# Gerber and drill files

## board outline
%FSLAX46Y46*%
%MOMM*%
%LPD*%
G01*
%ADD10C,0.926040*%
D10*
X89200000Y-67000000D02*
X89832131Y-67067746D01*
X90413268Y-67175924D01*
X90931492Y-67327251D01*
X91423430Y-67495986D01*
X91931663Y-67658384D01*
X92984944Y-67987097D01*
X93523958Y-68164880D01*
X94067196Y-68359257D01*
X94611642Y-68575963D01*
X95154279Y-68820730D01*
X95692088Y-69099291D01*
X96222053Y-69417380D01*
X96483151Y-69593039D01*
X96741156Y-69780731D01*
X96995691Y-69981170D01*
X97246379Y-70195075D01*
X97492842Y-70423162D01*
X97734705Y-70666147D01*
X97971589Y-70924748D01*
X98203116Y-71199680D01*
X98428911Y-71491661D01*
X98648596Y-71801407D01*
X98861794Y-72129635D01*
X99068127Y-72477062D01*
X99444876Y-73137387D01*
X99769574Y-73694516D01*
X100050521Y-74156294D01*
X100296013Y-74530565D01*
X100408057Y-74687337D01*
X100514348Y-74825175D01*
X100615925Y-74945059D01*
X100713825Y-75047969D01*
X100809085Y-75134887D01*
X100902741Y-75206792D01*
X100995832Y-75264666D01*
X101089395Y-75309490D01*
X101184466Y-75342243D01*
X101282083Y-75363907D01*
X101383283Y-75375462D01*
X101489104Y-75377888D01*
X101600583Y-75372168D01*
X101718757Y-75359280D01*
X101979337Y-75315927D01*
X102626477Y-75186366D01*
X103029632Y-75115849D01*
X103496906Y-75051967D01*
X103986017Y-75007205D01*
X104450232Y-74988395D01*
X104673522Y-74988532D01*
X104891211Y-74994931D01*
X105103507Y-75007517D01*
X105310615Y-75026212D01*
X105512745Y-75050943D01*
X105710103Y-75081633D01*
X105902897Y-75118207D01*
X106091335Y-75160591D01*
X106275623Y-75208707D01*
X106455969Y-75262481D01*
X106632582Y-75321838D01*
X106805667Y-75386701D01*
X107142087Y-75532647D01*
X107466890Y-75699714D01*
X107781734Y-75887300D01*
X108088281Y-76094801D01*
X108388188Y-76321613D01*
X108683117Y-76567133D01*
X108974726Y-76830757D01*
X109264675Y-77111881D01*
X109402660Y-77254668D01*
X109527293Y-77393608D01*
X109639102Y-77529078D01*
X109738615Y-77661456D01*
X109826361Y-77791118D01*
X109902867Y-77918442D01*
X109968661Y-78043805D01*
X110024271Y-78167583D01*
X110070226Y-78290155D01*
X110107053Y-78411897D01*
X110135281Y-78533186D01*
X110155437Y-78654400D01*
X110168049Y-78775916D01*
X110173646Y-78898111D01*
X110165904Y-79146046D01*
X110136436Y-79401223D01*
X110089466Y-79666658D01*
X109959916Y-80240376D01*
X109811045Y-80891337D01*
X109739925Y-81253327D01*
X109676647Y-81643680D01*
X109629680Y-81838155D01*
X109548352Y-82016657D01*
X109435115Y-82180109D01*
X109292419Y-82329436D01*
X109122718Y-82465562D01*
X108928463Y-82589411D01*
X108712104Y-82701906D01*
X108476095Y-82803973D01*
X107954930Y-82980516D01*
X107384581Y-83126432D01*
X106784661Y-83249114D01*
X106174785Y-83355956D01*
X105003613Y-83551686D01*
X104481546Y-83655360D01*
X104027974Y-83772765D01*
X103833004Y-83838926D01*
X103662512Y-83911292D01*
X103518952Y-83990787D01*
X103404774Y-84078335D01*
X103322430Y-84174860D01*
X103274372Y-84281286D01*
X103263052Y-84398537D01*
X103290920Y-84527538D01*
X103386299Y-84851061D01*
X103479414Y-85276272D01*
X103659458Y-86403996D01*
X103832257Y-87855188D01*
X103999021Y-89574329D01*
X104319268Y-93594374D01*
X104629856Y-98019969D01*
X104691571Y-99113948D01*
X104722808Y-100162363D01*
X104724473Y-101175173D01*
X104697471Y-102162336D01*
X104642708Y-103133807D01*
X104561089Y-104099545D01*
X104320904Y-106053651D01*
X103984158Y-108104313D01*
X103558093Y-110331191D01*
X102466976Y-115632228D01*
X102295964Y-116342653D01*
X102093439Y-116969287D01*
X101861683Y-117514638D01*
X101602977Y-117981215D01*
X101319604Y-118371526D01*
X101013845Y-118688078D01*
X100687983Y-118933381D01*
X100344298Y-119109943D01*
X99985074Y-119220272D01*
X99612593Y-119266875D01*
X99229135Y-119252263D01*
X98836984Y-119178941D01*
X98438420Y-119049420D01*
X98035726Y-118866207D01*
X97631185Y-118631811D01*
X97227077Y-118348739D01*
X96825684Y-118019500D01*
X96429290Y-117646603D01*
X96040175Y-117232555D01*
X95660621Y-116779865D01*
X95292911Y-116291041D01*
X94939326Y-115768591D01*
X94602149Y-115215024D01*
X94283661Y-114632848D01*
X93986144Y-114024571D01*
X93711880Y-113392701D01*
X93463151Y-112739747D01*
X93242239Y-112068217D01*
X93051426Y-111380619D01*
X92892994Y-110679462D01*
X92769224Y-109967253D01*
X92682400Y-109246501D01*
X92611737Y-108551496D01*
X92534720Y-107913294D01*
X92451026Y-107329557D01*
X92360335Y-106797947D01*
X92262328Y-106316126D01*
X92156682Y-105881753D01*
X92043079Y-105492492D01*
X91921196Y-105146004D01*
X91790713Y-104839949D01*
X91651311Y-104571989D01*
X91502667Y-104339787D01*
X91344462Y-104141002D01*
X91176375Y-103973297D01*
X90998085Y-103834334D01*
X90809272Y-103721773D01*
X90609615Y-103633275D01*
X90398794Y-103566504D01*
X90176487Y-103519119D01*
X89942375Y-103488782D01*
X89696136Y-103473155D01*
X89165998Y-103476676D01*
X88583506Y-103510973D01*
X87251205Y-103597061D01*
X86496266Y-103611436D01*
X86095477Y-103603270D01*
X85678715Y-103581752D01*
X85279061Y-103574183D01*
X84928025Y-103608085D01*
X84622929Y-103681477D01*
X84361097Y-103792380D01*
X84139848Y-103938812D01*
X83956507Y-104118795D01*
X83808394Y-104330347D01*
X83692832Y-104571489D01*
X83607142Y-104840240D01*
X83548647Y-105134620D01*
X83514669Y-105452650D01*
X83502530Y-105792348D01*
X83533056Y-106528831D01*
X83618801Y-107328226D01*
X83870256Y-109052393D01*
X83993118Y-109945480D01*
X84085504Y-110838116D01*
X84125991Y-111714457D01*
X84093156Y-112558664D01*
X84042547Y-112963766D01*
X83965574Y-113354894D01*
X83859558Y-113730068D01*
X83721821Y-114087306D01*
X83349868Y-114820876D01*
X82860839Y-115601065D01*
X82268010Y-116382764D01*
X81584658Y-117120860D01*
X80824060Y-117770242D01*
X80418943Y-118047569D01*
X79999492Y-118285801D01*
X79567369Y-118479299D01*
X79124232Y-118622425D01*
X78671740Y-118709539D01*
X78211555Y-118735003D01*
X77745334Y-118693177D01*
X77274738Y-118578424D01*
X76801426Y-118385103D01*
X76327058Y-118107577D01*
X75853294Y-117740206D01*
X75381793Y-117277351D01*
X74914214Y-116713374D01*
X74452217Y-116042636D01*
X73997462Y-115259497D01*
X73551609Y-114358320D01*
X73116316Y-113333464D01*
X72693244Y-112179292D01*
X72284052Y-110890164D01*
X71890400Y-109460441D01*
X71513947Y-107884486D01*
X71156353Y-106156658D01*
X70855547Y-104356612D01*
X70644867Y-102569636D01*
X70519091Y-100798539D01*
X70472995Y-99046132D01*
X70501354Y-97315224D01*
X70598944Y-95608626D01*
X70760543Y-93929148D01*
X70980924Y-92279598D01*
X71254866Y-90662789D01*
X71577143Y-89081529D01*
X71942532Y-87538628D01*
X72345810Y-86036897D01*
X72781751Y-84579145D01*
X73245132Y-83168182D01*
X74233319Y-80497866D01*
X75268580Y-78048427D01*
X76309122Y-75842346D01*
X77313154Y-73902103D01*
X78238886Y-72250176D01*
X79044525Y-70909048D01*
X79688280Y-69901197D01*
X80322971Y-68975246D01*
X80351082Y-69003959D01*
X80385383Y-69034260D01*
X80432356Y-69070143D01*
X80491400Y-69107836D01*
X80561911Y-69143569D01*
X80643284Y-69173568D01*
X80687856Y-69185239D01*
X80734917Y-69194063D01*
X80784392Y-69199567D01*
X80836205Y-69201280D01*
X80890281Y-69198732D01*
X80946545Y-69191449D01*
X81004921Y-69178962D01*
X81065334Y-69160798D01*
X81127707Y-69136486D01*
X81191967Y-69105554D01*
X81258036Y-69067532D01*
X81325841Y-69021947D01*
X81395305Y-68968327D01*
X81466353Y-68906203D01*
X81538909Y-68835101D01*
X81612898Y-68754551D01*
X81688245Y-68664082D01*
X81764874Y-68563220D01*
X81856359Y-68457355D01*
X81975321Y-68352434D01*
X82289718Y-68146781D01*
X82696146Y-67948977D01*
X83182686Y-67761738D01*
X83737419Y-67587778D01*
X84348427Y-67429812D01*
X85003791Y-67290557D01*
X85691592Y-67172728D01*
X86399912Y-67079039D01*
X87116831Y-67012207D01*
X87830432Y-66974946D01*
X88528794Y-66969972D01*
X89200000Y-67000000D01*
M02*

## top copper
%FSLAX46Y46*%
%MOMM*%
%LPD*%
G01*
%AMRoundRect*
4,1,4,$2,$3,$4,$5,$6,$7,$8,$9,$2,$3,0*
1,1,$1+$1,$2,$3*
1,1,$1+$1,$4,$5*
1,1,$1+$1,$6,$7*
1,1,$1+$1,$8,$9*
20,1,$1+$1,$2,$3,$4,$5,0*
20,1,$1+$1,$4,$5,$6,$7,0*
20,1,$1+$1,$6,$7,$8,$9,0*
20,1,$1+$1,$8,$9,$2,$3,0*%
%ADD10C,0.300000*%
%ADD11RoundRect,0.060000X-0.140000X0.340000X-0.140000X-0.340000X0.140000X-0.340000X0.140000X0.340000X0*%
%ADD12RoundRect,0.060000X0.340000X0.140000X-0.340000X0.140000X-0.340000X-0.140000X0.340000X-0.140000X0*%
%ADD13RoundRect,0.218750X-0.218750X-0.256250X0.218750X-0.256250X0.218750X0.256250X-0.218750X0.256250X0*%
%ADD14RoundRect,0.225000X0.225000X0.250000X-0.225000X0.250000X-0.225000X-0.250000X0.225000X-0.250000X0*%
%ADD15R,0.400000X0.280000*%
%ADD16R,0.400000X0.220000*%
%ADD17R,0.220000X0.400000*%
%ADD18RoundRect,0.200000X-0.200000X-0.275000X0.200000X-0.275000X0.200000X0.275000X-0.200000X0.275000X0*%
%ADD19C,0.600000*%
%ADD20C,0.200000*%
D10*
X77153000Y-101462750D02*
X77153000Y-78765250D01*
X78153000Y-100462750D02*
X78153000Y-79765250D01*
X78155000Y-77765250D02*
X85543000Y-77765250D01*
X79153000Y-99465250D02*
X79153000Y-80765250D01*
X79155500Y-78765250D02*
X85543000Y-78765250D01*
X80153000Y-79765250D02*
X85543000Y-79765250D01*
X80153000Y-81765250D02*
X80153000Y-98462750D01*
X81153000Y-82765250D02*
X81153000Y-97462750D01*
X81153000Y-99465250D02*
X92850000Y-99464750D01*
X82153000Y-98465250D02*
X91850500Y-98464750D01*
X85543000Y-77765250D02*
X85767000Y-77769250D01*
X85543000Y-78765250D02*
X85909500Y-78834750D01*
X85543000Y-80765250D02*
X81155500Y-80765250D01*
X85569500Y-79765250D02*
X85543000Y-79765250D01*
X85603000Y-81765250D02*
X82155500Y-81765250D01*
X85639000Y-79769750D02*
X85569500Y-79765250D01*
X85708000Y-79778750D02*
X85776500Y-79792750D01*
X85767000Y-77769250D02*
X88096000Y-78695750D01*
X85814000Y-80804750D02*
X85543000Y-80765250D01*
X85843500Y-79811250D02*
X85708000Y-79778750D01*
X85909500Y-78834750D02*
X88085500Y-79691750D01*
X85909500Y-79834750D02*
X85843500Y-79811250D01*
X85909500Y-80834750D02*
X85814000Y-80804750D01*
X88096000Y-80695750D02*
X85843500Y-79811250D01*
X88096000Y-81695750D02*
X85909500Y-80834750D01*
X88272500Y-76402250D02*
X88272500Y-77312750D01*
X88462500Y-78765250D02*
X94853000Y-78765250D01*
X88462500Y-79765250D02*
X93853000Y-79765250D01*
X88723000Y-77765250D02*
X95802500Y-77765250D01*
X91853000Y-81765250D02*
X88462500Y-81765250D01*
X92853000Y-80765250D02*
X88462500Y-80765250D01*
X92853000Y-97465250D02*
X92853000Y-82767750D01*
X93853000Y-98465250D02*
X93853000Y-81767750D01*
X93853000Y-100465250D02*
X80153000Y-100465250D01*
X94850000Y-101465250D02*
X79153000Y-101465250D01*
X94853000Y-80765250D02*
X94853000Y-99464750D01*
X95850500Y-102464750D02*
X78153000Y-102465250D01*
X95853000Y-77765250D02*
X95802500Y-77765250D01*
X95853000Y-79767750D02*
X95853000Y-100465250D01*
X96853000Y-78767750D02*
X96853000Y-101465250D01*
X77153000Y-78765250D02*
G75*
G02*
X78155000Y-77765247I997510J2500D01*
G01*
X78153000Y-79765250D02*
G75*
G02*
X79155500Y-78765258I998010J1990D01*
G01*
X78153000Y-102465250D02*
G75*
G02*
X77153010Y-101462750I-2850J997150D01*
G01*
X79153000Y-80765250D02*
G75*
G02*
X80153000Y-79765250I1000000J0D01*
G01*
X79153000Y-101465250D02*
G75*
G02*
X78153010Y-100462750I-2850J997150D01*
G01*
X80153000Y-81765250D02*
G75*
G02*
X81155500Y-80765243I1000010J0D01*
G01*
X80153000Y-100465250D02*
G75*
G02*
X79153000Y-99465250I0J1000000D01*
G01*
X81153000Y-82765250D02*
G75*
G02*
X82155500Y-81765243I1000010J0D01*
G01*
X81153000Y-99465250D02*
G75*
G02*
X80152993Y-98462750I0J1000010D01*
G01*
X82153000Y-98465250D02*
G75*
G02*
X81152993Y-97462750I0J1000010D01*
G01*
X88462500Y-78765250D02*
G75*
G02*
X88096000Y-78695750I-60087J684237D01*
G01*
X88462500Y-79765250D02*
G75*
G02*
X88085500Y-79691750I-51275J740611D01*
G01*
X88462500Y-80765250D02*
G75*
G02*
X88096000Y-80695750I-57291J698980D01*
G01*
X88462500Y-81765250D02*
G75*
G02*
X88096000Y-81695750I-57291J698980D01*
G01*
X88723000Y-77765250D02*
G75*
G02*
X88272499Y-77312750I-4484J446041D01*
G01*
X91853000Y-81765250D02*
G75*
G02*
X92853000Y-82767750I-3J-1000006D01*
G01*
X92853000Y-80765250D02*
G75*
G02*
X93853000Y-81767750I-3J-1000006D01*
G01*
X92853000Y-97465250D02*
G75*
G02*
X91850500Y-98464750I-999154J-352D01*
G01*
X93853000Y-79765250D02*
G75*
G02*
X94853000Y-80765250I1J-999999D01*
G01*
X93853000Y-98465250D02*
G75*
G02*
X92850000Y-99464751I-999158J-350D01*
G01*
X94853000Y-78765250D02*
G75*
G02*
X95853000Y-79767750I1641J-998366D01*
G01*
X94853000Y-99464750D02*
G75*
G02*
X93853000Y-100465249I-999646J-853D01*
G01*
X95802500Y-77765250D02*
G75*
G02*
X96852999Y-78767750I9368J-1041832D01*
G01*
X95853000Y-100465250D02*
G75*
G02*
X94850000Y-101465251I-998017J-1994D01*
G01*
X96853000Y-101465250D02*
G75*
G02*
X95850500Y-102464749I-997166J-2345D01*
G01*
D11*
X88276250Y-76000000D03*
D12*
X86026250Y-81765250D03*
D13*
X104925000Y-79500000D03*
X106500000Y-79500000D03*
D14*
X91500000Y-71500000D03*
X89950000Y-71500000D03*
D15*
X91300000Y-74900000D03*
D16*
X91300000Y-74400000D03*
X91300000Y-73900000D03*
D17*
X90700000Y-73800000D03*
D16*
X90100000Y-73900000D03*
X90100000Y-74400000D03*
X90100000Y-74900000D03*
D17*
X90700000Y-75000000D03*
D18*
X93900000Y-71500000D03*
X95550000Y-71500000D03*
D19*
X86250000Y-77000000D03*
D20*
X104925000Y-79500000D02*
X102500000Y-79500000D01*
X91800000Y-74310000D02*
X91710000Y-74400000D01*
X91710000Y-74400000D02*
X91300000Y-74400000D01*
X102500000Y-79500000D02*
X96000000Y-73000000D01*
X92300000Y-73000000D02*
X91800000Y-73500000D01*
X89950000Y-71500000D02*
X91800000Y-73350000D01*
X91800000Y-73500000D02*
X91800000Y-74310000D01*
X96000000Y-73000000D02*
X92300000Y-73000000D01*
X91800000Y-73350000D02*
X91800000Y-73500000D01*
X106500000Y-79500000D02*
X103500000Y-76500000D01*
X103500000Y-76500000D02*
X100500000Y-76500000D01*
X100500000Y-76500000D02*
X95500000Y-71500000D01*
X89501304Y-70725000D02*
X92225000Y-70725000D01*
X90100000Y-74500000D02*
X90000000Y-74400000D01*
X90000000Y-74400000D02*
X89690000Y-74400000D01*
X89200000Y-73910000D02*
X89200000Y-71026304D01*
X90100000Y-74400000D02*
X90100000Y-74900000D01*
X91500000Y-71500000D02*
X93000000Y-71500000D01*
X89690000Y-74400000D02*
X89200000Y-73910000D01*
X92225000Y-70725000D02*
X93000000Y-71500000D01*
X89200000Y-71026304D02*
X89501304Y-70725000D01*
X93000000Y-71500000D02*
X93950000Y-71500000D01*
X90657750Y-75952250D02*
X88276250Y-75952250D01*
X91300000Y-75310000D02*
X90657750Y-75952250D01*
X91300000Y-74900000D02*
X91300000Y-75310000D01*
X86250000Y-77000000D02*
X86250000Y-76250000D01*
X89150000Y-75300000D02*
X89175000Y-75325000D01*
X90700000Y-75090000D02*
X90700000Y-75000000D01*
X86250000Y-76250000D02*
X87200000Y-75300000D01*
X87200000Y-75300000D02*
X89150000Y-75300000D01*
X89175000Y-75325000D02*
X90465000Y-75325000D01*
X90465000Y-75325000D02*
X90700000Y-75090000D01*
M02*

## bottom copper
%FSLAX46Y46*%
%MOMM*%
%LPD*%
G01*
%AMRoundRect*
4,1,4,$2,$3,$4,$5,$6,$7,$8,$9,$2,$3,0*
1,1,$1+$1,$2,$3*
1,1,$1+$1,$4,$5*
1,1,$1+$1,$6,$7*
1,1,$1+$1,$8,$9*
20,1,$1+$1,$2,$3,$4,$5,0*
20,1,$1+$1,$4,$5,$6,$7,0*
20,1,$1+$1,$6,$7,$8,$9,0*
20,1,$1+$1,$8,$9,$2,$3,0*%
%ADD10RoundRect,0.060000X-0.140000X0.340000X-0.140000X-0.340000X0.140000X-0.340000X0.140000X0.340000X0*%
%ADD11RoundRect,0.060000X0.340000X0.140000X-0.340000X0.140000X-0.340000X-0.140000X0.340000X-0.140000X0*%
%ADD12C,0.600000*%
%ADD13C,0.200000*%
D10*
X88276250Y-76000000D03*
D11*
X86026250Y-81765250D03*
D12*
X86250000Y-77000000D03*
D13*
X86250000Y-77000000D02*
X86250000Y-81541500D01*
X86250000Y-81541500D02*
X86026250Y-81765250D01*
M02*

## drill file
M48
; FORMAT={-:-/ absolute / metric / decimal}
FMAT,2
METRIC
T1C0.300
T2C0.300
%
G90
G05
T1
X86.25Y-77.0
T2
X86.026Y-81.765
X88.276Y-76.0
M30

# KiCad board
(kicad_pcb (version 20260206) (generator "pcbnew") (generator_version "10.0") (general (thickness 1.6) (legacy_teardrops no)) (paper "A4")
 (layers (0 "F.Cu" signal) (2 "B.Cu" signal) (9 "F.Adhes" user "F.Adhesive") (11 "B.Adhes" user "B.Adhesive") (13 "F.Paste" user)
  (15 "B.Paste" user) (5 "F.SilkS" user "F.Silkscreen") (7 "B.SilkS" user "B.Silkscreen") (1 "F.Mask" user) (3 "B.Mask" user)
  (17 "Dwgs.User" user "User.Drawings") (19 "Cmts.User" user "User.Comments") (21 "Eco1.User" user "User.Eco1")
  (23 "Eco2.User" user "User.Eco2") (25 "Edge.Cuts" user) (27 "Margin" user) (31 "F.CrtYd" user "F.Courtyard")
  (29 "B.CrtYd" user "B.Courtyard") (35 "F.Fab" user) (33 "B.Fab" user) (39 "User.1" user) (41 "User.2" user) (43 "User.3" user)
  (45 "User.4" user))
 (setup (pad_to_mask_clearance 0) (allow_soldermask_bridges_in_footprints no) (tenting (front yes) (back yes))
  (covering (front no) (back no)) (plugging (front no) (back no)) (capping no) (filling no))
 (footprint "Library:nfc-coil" (layer "F.Cu") (at 87.12625 90.65 180)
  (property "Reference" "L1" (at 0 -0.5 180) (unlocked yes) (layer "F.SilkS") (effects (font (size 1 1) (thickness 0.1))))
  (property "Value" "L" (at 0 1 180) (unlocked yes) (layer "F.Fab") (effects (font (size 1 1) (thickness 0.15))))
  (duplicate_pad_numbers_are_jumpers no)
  (fp_line (start 9.97325 -10.81275) (end 9.97325 11.88475) (stroke (width 0.3) (type default)) (layer "F.Cu"))
  (fp_line (start 8.97325 -9.81275) (end 8.97325 10.88475) (stroke (width 0.3) (type default)) (layer "F.Cu"))
  (fp_line (start 8.97125 12.88475) (end 1.58325 12.88475) (stroke (width 0.3) (type default)) (layer "F.Cu"))
  (fp_line (start 7.97325 -8.81525) (end 7.97325 9.88475) (stroke (width 0.3) (type default)) (layer "F.Cu"))
  (fp_line (start 7.97075 11.88475) (end 1.58325 11.88475) (stroke (width 0.3) (type default)) (layer "F.Cu"))
  (fp_line (start 6.97325 10.88475) (end 1.58325 10.88475) (stroke (width 0.3) (type default)) (layer "F.Cu"))
  (fp_line (start 6.97325 8.88475) (end 6.97325 -7.81275) (stroke (width 0.3) (type default)) (layer "F.Cu"))
  (fp_line (start 5.97325 7.88475) (end 5.97325 -6.81275) (stroke (width 0.3) (type default)) (layer "F.Cu"))
  (fp_line (start 5.97325 -8.81525) (end -5.72375 -8.81475) (stroke (width 0.3) (type default)) (layer "F.Cu"))
  (fp_line (start 4.97325 -7.81525) (end -4.72425 -7.81475) (stroke (width 0.3) (type default)) (layer "F.Cu"))
  (fp_line (start 1.58325 12.88475) (end 1.35925 12.88075) (stroke (width 0.3) (type default)) (layer "F.Cu"))
  (fp_line (start 1.58325 11.88475) (end 1.21675 11.81525) (stroke (width 0.3) (type default)) (layer "F.Cu"))
  (fp_line (start 1.58325 9.88475) (end 5.97075 9.88475) (stroke (width 0.3) (type default)) (layer "F.Cu"))
  (fp_line (start 1.55675 10.88475) (end 1.58325 10.88475) (stroke (width 0.3) (type default)) (layer "F.Cu"))
  (fp_line (start 1.52325 8.88475) (end 4.97075 8.88475) (stroke (width 0.3) (type default)) (layer "F.Cu"))
  (fp_line (start 1.48725 10.88025) (end 1.55675 10.88475) (stroke (width 0.3) (type default)) (layer "F.Cu"))
  (fp_line (start 1.41825 10.87125) (end 1.34975 10.85725) (stroke (width 0.3) (type default)) (layer "F.Cu"))
  (fp_line (start 1.35925 12.88075) (end -0.96975 11.95425) (stroke (width 0.3) (type default)) (layer "F.Cu"))
  (fp_line (start 1.31225 9.84525) (end 1.58325 9.88475) (stroke (width 0.3) (type default)) (layer "F.Cu"))
  (fp_line (start 1.28275 10.83875) (end 1.41825 10.87125) (stroke (width 0.3) (type default)) (layer "F.Cu"))
  (fp_line (start 1.21675 11.81525) (end -0.95925 10.95825) (stroke (width 0.3) (type default)) (layer "F.Cu"))
  (fp_line (start 1.21675 10.81525) (end 1.28275 10.83875) (stroke (width 0.3) (type default)) (layer "F.Cu"))
  (fp_line (start 1.21675 9.81525) (end 1.31225 9.84525) (stroke (width 0.3) (type default)) (layer "F.Cu"))
  (fp_line (start -0.96975 9.95425) (end 1.28275 10.83875) (stroke (width 0.3) (type default)) (layer "F.Cu"))
  (fp_line (start -0.96975 8.95425) (end 1.21675 9.81525) (stroke (width 0.3) (type default)) (layer "F.Cu"))
  (fp_line (start -1.14625 14.24775) (end -1.14625 13.33725) (stroke (width 0.3) (type default)) (layer "F.Cu"))
  (fp_line (start -1.33625 11.88475) (end -7.72675 11.88475) (stroke (width 0.3) (type default)) (layer "F.Cu"))
  (fp_line (start -1.33625 10.88475) (end -6.72675 10.88475) (stroke (width 0.3) (type default)) (layer "F.Cu"))
  (fp_line (start -1.59675 12.88475) (end -8.67625 12.88475) (stroke (width 0.3) (type default)) (layer "F.Cu"))
  (fp_line (start -4.72675 8.88475) (end -1.33625 8.88475) (stroke (width 0.3) (type default)) (layer "F.Cu"))
  (fp_line (start -5.72675 9.88475) (end -1.33625 9.88475) (stroke (width 0.3) (type default)) (layer "F.Cu"))
  (fp_line (start -5.72675 -6.81525) (end -5.72675 7.88225) (stroke (width 0.3) (type default)) (layer "F.Cu"))
  (fp_line (start -6.72675 -7.81525) (end -6.72675 8.88225) (stroke (width 0.3) (type default)) (layer "F.Cu"))
  (fp_line (start -6.72675 -9.81525) (end 6.97325 -9.81525) (stroke (width 0.3) (type default)) (layer "F.Cu"))
  (fp_line (start -7.72375 -10.81525) (end 7.97325 -10.81525) (stroke (width 0.3) (type default)) (layer "F.Cu"))
  (fp_line (start -7.72675 9.88475) (end -7.72675 -8.81475) (stroke (width 0.3) (type default)) (layer "F.Cu"))
  (fp_line (start -8.72425 -11.81475) (end 8.97325 -11.81525) (stroke (width 0.3) (type default)) (layer "F.Cu"))
  (fp_line (start -8.72675 12.88475) (end -8.67625 12.88475) (stroke (width 0.3) (type default)) (layer "F.Cu"))
  (fp_line (start -8.72675 10.88225) (end -8.72675 -9.81525) (stroke (width 0.3) (type default)) (layer "F.Cu"))
  (fp_line (start -9.72675 11.88225) (end -9.72675 -10.81525) (stroke (width 0.3) (type default)) (layer "F.Cu"))
  (fp_arc (start 9.97325 11.88475) (mid 9.680384 12.593298) (end 8.97125 12.88475) (stroke (width 0.3) (type default)) (layer "F.Cu"))
  (fp_arc (start 8.97325 10.88475) (mid 8.68006 11.593327) (end 7.97075 11.88475) (stroke (width 0.3) (type default)) (layer "F.Cu"))
  (fp_arc (start 8.97325 -11.81525) (mid 9.682152 -11.522237) (end 9.97325 -10.81275) (stroke (width 0.3) (type default)) (layer "F.Cu"))
  (fp_arc (start 7.97325 9.88475) (mid 7.680357 10.591857) (end 6.97325 10.88475) (stroke (width 0.3) (type default)) (layer "F.Cu"))
  (fp_arc (start 7.97325 -10.81525) (mid 8.682152 -10.522237) (end 8.97325 -9.81275) (stroke (width 0.3) (type default)) (layer "F.Cu"))
  (fp_arc (start 6.97325 8.88475) (mid 6.679472 9.59274) (end 5.97075 9.88475) (stroke (width 0.3) (type default)) (layer "F.Cu"))
  (fp_arc (start 6.97325 -9.81525) (mid 7.680357 -9.522357) (end 7.97325 -8.81525) (stroke (width 0.3) (type default)) (layer "F.Cu"))
  (fp_arc (start 5.97325 7.88475) (mid 5.679472 8.59274) (end 4.97075 8.88475) (stroke (width 0.3) (type default)) (layer "F.Cu"))
  (fp_arc (start 5.97325 -8.81525) (mid 6.68124 -8.521472) (end 6.97325 -7.81275) (stroke (width 0.3) (type default)) (layer "F.Cu"))
  (fp_arc (start 4.97325 -7.81525) (mid 5.68124 -7.521472) (end 5.97325 -6.81275) (stroke (width 0.3) (type default)) (layer "F.Cu"))
  (fp_arc (start -1.33625 11.88475) (mid -1.148183 11.894145) (end -0.96975 11.95425) (stroke (width 0.3) (type default)) (layer "F.Cu"))
  (fp_arc (start -1.33625 10.88475) (mid -1.14293 10.896693) (end -0.95925 10.95825) (stroke (width 0.3) (type default)) (layer "F.Cu"))
  (fp_arc (start -1.33625 9.88475) (mid -1.148314 9.894682) (end -0.96975 9.95425) (stroke (width 0.3) (type default)) (layer "F.Cu"))
  (fp_arc (start -1.33625 8.88475) (mid -1.148314 8.894682) (end -0.96975 8.95425) (stroke (width 0.3) (type default)) (layer "F.Cu"))
  (fp_arc (start -1.59675 12.88475) (mid -1.276158 13.016072) (end -1.14625 13.33725) (stroke (width 0.3) (type default)) (layer "F.Cu"))
  (fp_arc (start -4.72675 8.88475) (mid -5.43474 8.590972) (end -5.72675 7.88225) (stroke (width 0.3) (type default)) (layer "F.Cu"))
  (fp_arc (start -5.72675 9.88475) (mid -6.43474 9.590972) (end -6.72675 8.88225) (stroke (width 0.3) (type default)) (layer "F.Cu"))
  (fp_arc (start -5.72675 -6.81525) (mid -5.432972 -7.523241) (end -4.72425 -7.81475) (stroke (width 0.3) (type default)) (layer "F.Cu"))
  (fp_arc (start -6.72675 10.88475) (mid -7.433857 10.591857) (end -7.72675 9.88475) (stroke (width 0.3) (type default)) (layer "F.Cu"))
  (fp_arc (start -6.72675 -7.81525) (mid -6.432795 -8.523417) (end -5.72375 -8.81475) (stroke (width 0.3) (type default)) (layer "F.Cu"))
  (fp_arc (start -7.72675 11.88475) (mid -8.435149 11.59153) (end -8.72675 10.88225) (stroke (width 0.3) (type default)) (layer "F.Cu"))
  (fp_arc (start -7.72675 -8.81475) (mid -7.434064 -9.522357) (end -6.72675 -9.81525) (stroke (width 0.3) (type default)) (layer "F.Cu"))
  (fp_arc (start -8.67625 12.88475) (mid -9.404886 12.596679) (end -9.72675 11.88225) (stroke (width 0.3) (type default)) (layer "F.Cu"))
  (fp_arc (start -8.72675 -9.81525) (mid -8.433383 -10.524004) (end -7.72375 -10.81525) (stroke (width 0.3) (type default)) (layer "F.Cu"))
  (fp_arc (start -9.72675 -10.81525) (mid -9.433559 -11.523828) (end -8.72425 -11.81475) (stroke (width 0.3) (type default)) (layer "F.Cu"))
  (pad "1" thru_hole roundrect (at -1.15 14.65 270) (size 0.8 0.4) (drill 0.3) (layers "*.Cu" "*.Mask") (remove_unused_layers no)
   (roundrect_rratio 0.15) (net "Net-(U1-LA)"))
  (pad "2" thru_hole roundrect (at 1.1 8.88475 180) (size 0.8 0.4) (drill 0.3) (layers "*.Cu" "*.Mask") (remove_unused_layers no)
   (roundrect_rratio 0.15) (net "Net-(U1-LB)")))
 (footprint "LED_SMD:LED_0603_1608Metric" (layer "F.Cu") (at 105.7125 79.5)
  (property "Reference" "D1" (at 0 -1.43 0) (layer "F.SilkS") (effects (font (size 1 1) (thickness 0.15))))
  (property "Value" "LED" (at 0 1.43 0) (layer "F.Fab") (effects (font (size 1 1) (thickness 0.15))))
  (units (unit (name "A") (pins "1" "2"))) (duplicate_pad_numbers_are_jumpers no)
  (pad "1" smd roundrect (at -0.7875 0) (size 0.875 0.95) (layers "F.Cu" "F.Mask" "F.Paste") (roundrect_rratio 0.25) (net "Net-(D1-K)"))
  (pad "2" smd roundrect (at 0.7875 0) (size 0.875 0.95) (layers "F.Cu" "F.Mask" "F.Paste") (roundrect_rratio 0.25) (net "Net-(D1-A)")))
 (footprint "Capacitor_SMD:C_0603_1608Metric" (layer "F.Cu") (at 90.725 71.5 180)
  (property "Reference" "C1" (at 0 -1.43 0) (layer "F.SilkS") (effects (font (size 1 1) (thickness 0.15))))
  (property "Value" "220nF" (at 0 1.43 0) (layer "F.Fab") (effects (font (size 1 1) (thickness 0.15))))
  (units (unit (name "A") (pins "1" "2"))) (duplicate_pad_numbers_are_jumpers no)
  (pad "1" smd roundrect (at -0.775 0 180) (size 0.9 0.95) (layers "F.Cu" "F.Mask" "F.Paste") (roundrect_rratio 0.25) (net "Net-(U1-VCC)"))
  (pad "2" smd roundrect (at 0.775 0 180) (size 0.9 0.95) (layers "F.Cu" "F.Mask" "F.Paste") (roundrect_rratio 0.25) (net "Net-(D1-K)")))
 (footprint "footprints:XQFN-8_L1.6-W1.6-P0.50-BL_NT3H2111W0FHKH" (layer "F.Cu") (at 90.7 74.4 180)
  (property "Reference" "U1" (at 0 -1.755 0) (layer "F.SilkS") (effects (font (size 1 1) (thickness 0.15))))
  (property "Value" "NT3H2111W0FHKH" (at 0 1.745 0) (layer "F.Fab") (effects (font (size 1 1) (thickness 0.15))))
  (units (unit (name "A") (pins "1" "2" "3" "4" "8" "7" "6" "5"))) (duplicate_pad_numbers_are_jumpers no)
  (pad "1" smd rect (at -0.6 -0.5 180) (size 0.4 0.28) (layers "F.Cu" "F.Mask" "F.Paste") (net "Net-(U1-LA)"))
  (pad "2" smd rect (at -0.6 0 180) (size 0.4 0.22) (layers "F.Cu" "F.Mask" "F.Paste") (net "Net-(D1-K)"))
  (pad "3" smd rect (at -0.6 0.5 180) (size 0.4 0.22) (layers "F.Cu" "F.Mask" "F.Paste") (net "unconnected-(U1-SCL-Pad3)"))
  (pad "4" smd rect (at 0 0.6 270) (size 0.4 0.22) (layers "F.Cu" "F.Mask" "F.Paste") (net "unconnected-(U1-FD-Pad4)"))
  (pad "5" smd rect (at 0.6 0.5 180) (size 0.4 0.22) (layers "F.Cu" "F.Mask" "F.Paste") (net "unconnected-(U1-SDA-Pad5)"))
  (pad "6" smd rect (at 0.6 0 180) (size 0.4 0.22) (layers "F.Cu" "F.Mask" "F.Paste") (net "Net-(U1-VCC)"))
  (pad "7" smd rect (at 0.6 -0.5 180) (size 0.4 0.22) (layers "F.Cu" "F.Mask" "F.Paste") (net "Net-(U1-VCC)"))
  (pad "8" smd rect (at 0 -0.6 270) (size 0.4 0.22) (layers "F.Cu" "F.Mask" "F.Paste") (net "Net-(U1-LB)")))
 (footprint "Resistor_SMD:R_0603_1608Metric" (layer "F.Cu") (at 94.725 71.5)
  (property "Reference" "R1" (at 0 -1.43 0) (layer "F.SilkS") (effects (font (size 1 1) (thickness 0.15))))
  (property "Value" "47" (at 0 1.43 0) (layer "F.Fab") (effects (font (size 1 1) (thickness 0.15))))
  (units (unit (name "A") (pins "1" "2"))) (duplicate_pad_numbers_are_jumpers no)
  (pad "1" smd roundrect (at -0.825 0) (size 0.8 0.95) (layers "F.Cu" "F.Mask" "F.Paste") (roundrect_rratio 0.25) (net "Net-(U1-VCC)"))
  (pad "2" smd roundrect (at 0.825 0) (size 0.8 0.95) (layers "F.Cu" "F.Mask" "F.Paste") (roundrect_rratio 0.25) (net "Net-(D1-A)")))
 (gr_poly
  (pts (xy 89.2 67) (xy 89.832131 67.067746) (xy 90.413268 67.175924) (xy 90.931492 67.327251) (xy 91.42343 67.495986)
   (xy 91.931663 67.658384) (xy 92.984944 67.987097) (xy 93.523958 68.16488) (xy 94.067196 68.359257) (xy 94.611642 68.575963)
   (xy 95.154279 68.82073) (xy 95.692088 69.099291) (xy 96.222053 69.41738) (xy 96.483151 69.593039) (xy 96.741156 69.780731)
   (xy 96.995691 69.98117) (xy 97.246379 70.195075) (xy 97.492842 70.423162) (xy 97.734705 70.666147) (xy 97.971589 70.924748)
   (xy 98.203116 71.19968) (xy 98.428911 71.491661) (xy 98.648596 71.801407) (xy 98.861794 72.129635) (xy 99.068127 72.477062)
   (xy 99.444876 73.137387) (xy 99.769574 73.694516) (xy 100.050521 74.156294) (xy 100.296013 74.530565) (xy 100.408057 74.687337)
   (xy 100.514348 74.825175) (xy 100.615925 74.945059) (xy 100.713825 75.047969) (xy 100.809085 75.134887) (xy 100.902741 75.206792)
   (xy 100.995832 75.264666) (xy 101.089395 75.30949) (xy 101.184466 75.342243) (xy 101.282083 75.363907) (xy 101.383283 75.375462)
   (xy 101.489104 75.377888) (xy 101.600583 75.372168) (xy 101.718757 75.35928) (xy 101.979337 75.315927) (xy 102.626477 75.186366)
   (xy 103.029632 75.115849) (xy 103.496906 75.051967) (xy 103.986017 75.007205) (xy 104.450232 74.988395) (xy 104.673522 74.988532)
   (xy 104.891211 74.994931) (xy 105.103507 75.007517) (xy 105.310615 75.026212) (xy 105.512745 75.050943) (xy 105.710103 75.081633)
   (xy 105.902897 75.118207) (xy 106.091335 75.160591) (xy 106.275623 75.208707) (xy 106.455969 75.262481) (xy 106.632582 75.321838)
   (xy 106.805667 75.386701) (xy 107.142087 75.532647) (xy 107.46689 75.699714) (xy 107.781734 75.8873) (xy 108.088281 76.094801)
   (xy 108.388188 76.321613) (xy 108.683117 76.567133) (xy 108.974726 76.830757) (xy 109.264675 77.111881) (xy 109.40266 77.254668)
   (xy 109.527293 77.393608) (xy 109.639102 77.529078) (xy 109.738615 77.661456) (xy 109.826361 77.791118) (xy 109.902867 77.918442)
   (xy 109.968661 78.043805) (xy 110.024271 78.167583) (xy 110.070226 78.290155) (xy 110.107053 78.411897) (xy 110.135281 78.533186)
   (xy 110.155437 78.6544) (xy 110.168049 78.775916) (xy 110.173646 78.898111) (xy 110.165904 79.146046) (xy 110.136436 79.401223)
   (xy 110.089466 79.666658) (xy 109.959916 80.240376) (xy 109.811045 80.891337) (xy 109.739925 81.253327) (xy 109.676647 81.64368)
   (xy 109.62968 81.838155) (xy 109.548352 82.016657) (xy 109.435115 82.180109) (xy 109.292419 82.329436) (xy 109.122718 82.465562)
   (xy 108.928463 82.589411) (xy 108.712104 82.701906) (xy 108.476095 82.803973) (xy 107.95493 82.980516) (xy 107.384581 83.126432)
   (xy 106.784661 83.249114) (xy 106.174785 83.355956) (xy 105.003613 83.551686) (xy 104.481546 83.65536) (xy 104.027974 83.772765)
   (xy 103.833004 83.838926) (xy 103.662512 83.911292) (xy 103.518952 83.990787) (xy 103.404774 84.078335) (xy 103.32243 84.17486)
   (xy 103.274372 84.281286) (xy 103.263052 84.398537) (xy 103.29092 84.527538) (xy 103.386299 84.851061) (xy 103.479414 85.276272)
   (xy 103.659458 86.403996) (xy 103.832257 87.855188) (xy 103.999021 89.574329) (xy 104.319268 93.594374) (xy 104.629856 98.019969)
   (xy 104.691571 99.113948) (xy 104.722808 100.162363) (xy 104.724473 101.175173) (xy 104.697471 102.162336) (xy 104.642708 103.133807)
   (xy 104.561089 104.099545) (xy 104.320904 106.053651) (xy 103.984158 108.104313) (xy 103.558093 110.331191) (xy 102.466976 115.632228)
   (xy 102.295964 116.342653) (xy 102.093439 116.969287) (xy 101.861683 117.514638) (xy 101.602977 117.981215) (xy 101.319604 118.371526)
   (xy 101.013845 118.688078) (xy 100.687983 118.933381) (xy 100.344298 119.109943) (xy 99.985074 119.220272) (xy 99.612593 119.266875)
   (xy 99.229135 119.252263) (xy 98.836984 119.178941) (xy 98.43842 119.04942) (xy 98.035726 118.866207) (xy 97.631185 118.631811)
   (xy 97.227077 118.348739) (xy 96.825684 118.0195) (xy 96.42929 117.646603) (xy 96.040175 117.232555) (xy 95.660621 116.779865)
   (xy 95.292911 116.291041) (xy 94.939326 115.768591) (xy 94.602149 115.215024) (xy 94.283661 114.632848) (xy 93.986144 114.024571)
   (xy 93.71188 113.392701) (xy 93.463151 112.739747) (xy 93.242239 112.068217) (xy 93.051426 111.380619) (xy 92.892994 110.679462)
   (xy 92.769224 109.967253) (xy 92.6824 109.246501) (xy 92.611737 108.551496) (xy 92.53472 107.913294) (xy 92.451026 107.329557)
   (xy 92.360335 106.797947) (xy 92.262328 106.316126) (xy 92.156682 105.881753) (xy 92.043079 105.492492) (xy 91.921196 105.146004)
   (xy 91.790713 104.839949) (xy 91.651311 104.571989) (xy 91.502667 104.339787) (xy 91.344462 104.141002) (xy 91.176375 103.973297)
   (xy 90.998085 103.834334) (xy 90.809272 103.721773) (xy 90.609615 103.633275) (xy 90.398794 103.566504) (xy 90.176487 103.519119)
   (xy 89.942375 103.488782) (xy 89.696136 103.473155) (xy 89.165998 103.476676) (xy 88.583506 103.510973) (xy 87.251205 103.597061)
   (xy 86.496266 103.611436) (xy 86.095477 103.60327) (xy 85.678715 103.581752) (xy 85.279061 103.574183) (xy 84.928025 103.608085)
   (xy 84.622929 103.681477) (xy 84.361097 103.79238) (xy 84.139848 103.938812) (xy 83.956507 104.118795) (xy 83.808394 104.330347)
   (xy 83.692832 104.571489) (xy 83.607142 104.84024) (xy 83.548647 105.13462) (xy 83.514669 105.45265) (xy 83.50253 105.792348)
   (xy 83.533056 106.528831) (xy 83.618801 107.328226) (xy 83.870256 109.052393) (xy 83.993118 109.94548) (xy 84.085504 110.838116)
   (xy 84.125991 111.714457) (xy 84.093156 112.558664) (xy 84.042547 112.963766) (xy 83.965574 113.354894) (xy 83.859558 113.730068)
   (xy 83.721821 114.087306) (xy 83.349868 114.820876) (xy 82.860839 115.601065) (xy 82.26801 116.382764) (xy 81.584658 117.12086)
   (xy 80.82406 117.770242) (xy 80.418943 118.047569) (xy 79.999492 118.285801) (xy 79.567369 118.479299) (xy 79.124232 118.622425)
   (xy 78.67174 118.709539) (xy 78.211555 118.735003) (xy 77.745334 118.693177) (xy 77.274738 118.578424) (xy 76.801426 118.385103)
   (xy 76.327058 118.107577) (xy 75.853294 117.740206) (xy 75.381793 117.277351) (xy 74.914214 116.713374) (xy 74.452217 116.042636)
   (xy 73.997462 115.259497) (xy 73.551609 114.35832) (xy 73.116316 113.333464) (xy 72.693244 112.179292) (xy 72.284052 110.890164)
   (xy 71.8904 109.460441) (xy 71.513947 107.884486) (xy 71.156353 106.156658) (xy 70.855547 104.356612) (xy 70.644867 102.569636)
   (xy 70.519091 100.798539) (xy 70.472995 99.046132) (xy 70.501354 97.315224) (xy 70.598944 95.608626) (xy 70.760543 93.929148)
   (xy 70.980924 92.279598) (xy 71.254866 90.662789) (xy 71.577143 89.081529) (xy 71.942532 87.538628) (xy 72.34581 86.036897)
   (xy 72.781751 84.579145) (xy 73.245132 83.168182) (xy 74.233319 80.497866) (xy 75.26858 78.048427) (xy 76.309122 75.842346)
   (xy 77.313154 73.902103) (xy 78.238886 72.250176) (xy 79.044525 70.909048) (xy 79.68828 69.901197) (xy 80.322971 68.975246)
   (xy 80.351082 69.003959) (xy 80.385383 69.03426) (xy 80.432356 69.070143) (xy 80.4914 69.107836) (xy 80.561911 69.143569)
   (xy 80.643284 69.173568) (xy 80.687856 69.185239) (xy 80.734917 69.194063) (xy 80.784392 69.199567) (xy 80.836205 69.20128)
   (xy 80.890281 69.198732) (xy 80.946545 69.191449) (xy 81.004921 69.178962) (xy 81.065334 69.160798) (xy 81.127707 69.136486)
   (xy 81.191967 69.105554) (xy 81.258036 69.067532) (xy 81.325841 69.021947) (xy 81.395305 68.968327) (xy 81.466353 68.906203)
   (xy 81.538909 68.835101) (xy 81.612898 68.754551) (xy 81.688245 68.664082) (xy 81.764874 68.56322) (xy 81.856359 68.457355)
   (xy 81.975321 68.352434) (xy 82.289718 68.146781) (xy 82.696146 67.948977) (xy 83.182686 67.761738) (xy 83.737419 67.587778)
   (xy 84.348427 67.429812) (xy 85.003791 67.290557) (xy 85.691592 67.172728) (xy 86.399912 67.079039) (xy 87.116831 67.012207)
   (xy 87.830432 66.974946) (xy 88.528794 66.969972))
  (stroke (width 0.92604) (type solid)) (fill no) (layer "Edge.Cuts"))
 (segment (start 104.925 79.5) (end 102.5 79.5) (width 0.2) (layer "F.Cu") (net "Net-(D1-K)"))
 (segment (start 91.8 74.31) (end 91.71 74.4) (width 0.2) (layer "F.Cu") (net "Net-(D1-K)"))
 (segment (start 91.71 74.4) (end 91.3 74.4) (width 0.2) (layer "F.Cu") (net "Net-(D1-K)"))
 (segment (start 102.5 79.5) (end 96 73) (width 0.2) (layer "F.Cu") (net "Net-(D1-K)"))
 (segment (start 92.3 73) (end 91.8 73.5) (width 0.2) (layer "F.Cu") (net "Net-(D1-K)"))
 (segment (start 89.95 71.5) (end 91.8 73.35) (width 0.2) (layer "F.Cu") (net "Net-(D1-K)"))
 (segment (start 91.8 73.5) (end 91.8 74.31) (width 0.2) (layer "F.Cu") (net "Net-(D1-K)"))
 (segment (start 96 73) (end 92.3 73) (width 0.2) (layer "F.Cu") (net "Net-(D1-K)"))
 (segment (start 91.8 73.35) (end 91.8 73.5) (width 0.2) (layer "F.Cu") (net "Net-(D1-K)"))
 (segment (start 106.5 79.5) (end 103.5 76.5) (width 0.2) (layer "F.Cu") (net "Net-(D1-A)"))
 (segment (start 103.5 76.5) (end 100.5 76.5) (width 0.2) (layer "F.Cu") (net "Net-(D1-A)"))
 (segment (start 100.5 76.5) (end 95.5 71.5) (width 0.2) (layer "F.Cu") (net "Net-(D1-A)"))
 (segment (start 89.501304 70.725) (end 92.225 70.725) (width 0.2) (layer "F.Cu") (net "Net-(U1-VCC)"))
 (segment (start 90.1 74.5) (end 90 74.4) (width 0.2) (layer "F.Cu") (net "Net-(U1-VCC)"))
 (segment (start 90 74.4) (end 89.69 74.4) (width 0.2) (layer "F.Cu") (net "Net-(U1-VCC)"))
 (segment (start 89.2 73.91) (end 89.2 71.026304) (width 0.2) (layer "F.Cu") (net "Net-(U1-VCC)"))
 (segment (start 90.1 74.4) (end 90.1 74.9) (width 0.2) (layer "F.Cu") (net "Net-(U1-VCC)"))
 (segment (start 91.5 71.5) (end 93 71.5) (width 0.2) (layer "F.Cu") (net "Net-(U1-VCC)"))
 (segment (start 89.69 74.4) (end 89.2 73.91) (width 0.2) (layer "F.Cu") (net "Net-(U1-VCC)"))
 (segment (start 92.225 70.725) (end 93 71.5) (width 0.2) (layer "F.Cu") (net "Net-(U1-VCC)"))
 (segment (start 89.2 71.026304) (end 89.501304 70.725) (width 0.2) (layer "F.Cu") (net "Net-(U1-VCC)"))
 (segment (start 93 71.5) (end 93.95 71.5) (width 0.2) (layer "F.Cu") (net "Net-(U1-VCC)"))
 (segment (start 90.65775 75.95225) (end 88.27625 75.95225) (width 0.2) (layer "F.Cu") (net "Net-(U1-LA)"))
 (segment (start 91.3 75.31) (end 90.65775 75.95225) (width 0.2) (layer "F.Cu") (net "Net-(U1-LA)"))
 (segment (start 91.3 74.9) (end 91.3 75.31) (width 0.2) (layer "F.Cu") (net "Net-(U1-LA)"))
 (segment (start 86.25 77) (end 86.25 76.25) (width 0.2) (layer "F.Cu") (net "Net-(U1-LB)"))
 (segment (start 89.15 75.3) (end 89.175 75.325) (width 0.2) (layer "F.Cu") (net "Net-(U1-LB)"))
 (segment (start 90.7 75.09) (end 90.7 75) (width 0.2) (layer "F.Cu") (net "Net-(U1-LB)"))
 (segment (start 86.25 76.25) (end 87.2 75.3) (width 0.2) (layer "F.Cu") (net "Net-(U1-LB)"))
 (segment (start 87.2 75.3) (end 89.15 75.3) (width 0.2) (layer "F.Cu") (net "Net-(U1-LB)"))
 (segment (start 89.175 75.325) (end 90.465 75.325) (width 0.2) (layer "F.Cu") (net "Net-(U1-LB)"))
 (segment (start 90.465 75.325) (end 90.7 75.09) (width 0.2) (layer "F.Cu") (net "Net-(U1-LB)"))
 (via (at 86.25 77) (size 0.6) (drill 0.3) (layers "F.Cu" "B.Cu") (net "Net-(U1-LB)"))
 (segment (start 86.25 77) (end 86.25 81.5415) (width 0.2) (layer "B.Cu") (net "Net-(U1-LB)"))
 (segment (start 86.25 81.5415) (end 86.02625 81.76525) (width 0.2) (layer "B.Cu") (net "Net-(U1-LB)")))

